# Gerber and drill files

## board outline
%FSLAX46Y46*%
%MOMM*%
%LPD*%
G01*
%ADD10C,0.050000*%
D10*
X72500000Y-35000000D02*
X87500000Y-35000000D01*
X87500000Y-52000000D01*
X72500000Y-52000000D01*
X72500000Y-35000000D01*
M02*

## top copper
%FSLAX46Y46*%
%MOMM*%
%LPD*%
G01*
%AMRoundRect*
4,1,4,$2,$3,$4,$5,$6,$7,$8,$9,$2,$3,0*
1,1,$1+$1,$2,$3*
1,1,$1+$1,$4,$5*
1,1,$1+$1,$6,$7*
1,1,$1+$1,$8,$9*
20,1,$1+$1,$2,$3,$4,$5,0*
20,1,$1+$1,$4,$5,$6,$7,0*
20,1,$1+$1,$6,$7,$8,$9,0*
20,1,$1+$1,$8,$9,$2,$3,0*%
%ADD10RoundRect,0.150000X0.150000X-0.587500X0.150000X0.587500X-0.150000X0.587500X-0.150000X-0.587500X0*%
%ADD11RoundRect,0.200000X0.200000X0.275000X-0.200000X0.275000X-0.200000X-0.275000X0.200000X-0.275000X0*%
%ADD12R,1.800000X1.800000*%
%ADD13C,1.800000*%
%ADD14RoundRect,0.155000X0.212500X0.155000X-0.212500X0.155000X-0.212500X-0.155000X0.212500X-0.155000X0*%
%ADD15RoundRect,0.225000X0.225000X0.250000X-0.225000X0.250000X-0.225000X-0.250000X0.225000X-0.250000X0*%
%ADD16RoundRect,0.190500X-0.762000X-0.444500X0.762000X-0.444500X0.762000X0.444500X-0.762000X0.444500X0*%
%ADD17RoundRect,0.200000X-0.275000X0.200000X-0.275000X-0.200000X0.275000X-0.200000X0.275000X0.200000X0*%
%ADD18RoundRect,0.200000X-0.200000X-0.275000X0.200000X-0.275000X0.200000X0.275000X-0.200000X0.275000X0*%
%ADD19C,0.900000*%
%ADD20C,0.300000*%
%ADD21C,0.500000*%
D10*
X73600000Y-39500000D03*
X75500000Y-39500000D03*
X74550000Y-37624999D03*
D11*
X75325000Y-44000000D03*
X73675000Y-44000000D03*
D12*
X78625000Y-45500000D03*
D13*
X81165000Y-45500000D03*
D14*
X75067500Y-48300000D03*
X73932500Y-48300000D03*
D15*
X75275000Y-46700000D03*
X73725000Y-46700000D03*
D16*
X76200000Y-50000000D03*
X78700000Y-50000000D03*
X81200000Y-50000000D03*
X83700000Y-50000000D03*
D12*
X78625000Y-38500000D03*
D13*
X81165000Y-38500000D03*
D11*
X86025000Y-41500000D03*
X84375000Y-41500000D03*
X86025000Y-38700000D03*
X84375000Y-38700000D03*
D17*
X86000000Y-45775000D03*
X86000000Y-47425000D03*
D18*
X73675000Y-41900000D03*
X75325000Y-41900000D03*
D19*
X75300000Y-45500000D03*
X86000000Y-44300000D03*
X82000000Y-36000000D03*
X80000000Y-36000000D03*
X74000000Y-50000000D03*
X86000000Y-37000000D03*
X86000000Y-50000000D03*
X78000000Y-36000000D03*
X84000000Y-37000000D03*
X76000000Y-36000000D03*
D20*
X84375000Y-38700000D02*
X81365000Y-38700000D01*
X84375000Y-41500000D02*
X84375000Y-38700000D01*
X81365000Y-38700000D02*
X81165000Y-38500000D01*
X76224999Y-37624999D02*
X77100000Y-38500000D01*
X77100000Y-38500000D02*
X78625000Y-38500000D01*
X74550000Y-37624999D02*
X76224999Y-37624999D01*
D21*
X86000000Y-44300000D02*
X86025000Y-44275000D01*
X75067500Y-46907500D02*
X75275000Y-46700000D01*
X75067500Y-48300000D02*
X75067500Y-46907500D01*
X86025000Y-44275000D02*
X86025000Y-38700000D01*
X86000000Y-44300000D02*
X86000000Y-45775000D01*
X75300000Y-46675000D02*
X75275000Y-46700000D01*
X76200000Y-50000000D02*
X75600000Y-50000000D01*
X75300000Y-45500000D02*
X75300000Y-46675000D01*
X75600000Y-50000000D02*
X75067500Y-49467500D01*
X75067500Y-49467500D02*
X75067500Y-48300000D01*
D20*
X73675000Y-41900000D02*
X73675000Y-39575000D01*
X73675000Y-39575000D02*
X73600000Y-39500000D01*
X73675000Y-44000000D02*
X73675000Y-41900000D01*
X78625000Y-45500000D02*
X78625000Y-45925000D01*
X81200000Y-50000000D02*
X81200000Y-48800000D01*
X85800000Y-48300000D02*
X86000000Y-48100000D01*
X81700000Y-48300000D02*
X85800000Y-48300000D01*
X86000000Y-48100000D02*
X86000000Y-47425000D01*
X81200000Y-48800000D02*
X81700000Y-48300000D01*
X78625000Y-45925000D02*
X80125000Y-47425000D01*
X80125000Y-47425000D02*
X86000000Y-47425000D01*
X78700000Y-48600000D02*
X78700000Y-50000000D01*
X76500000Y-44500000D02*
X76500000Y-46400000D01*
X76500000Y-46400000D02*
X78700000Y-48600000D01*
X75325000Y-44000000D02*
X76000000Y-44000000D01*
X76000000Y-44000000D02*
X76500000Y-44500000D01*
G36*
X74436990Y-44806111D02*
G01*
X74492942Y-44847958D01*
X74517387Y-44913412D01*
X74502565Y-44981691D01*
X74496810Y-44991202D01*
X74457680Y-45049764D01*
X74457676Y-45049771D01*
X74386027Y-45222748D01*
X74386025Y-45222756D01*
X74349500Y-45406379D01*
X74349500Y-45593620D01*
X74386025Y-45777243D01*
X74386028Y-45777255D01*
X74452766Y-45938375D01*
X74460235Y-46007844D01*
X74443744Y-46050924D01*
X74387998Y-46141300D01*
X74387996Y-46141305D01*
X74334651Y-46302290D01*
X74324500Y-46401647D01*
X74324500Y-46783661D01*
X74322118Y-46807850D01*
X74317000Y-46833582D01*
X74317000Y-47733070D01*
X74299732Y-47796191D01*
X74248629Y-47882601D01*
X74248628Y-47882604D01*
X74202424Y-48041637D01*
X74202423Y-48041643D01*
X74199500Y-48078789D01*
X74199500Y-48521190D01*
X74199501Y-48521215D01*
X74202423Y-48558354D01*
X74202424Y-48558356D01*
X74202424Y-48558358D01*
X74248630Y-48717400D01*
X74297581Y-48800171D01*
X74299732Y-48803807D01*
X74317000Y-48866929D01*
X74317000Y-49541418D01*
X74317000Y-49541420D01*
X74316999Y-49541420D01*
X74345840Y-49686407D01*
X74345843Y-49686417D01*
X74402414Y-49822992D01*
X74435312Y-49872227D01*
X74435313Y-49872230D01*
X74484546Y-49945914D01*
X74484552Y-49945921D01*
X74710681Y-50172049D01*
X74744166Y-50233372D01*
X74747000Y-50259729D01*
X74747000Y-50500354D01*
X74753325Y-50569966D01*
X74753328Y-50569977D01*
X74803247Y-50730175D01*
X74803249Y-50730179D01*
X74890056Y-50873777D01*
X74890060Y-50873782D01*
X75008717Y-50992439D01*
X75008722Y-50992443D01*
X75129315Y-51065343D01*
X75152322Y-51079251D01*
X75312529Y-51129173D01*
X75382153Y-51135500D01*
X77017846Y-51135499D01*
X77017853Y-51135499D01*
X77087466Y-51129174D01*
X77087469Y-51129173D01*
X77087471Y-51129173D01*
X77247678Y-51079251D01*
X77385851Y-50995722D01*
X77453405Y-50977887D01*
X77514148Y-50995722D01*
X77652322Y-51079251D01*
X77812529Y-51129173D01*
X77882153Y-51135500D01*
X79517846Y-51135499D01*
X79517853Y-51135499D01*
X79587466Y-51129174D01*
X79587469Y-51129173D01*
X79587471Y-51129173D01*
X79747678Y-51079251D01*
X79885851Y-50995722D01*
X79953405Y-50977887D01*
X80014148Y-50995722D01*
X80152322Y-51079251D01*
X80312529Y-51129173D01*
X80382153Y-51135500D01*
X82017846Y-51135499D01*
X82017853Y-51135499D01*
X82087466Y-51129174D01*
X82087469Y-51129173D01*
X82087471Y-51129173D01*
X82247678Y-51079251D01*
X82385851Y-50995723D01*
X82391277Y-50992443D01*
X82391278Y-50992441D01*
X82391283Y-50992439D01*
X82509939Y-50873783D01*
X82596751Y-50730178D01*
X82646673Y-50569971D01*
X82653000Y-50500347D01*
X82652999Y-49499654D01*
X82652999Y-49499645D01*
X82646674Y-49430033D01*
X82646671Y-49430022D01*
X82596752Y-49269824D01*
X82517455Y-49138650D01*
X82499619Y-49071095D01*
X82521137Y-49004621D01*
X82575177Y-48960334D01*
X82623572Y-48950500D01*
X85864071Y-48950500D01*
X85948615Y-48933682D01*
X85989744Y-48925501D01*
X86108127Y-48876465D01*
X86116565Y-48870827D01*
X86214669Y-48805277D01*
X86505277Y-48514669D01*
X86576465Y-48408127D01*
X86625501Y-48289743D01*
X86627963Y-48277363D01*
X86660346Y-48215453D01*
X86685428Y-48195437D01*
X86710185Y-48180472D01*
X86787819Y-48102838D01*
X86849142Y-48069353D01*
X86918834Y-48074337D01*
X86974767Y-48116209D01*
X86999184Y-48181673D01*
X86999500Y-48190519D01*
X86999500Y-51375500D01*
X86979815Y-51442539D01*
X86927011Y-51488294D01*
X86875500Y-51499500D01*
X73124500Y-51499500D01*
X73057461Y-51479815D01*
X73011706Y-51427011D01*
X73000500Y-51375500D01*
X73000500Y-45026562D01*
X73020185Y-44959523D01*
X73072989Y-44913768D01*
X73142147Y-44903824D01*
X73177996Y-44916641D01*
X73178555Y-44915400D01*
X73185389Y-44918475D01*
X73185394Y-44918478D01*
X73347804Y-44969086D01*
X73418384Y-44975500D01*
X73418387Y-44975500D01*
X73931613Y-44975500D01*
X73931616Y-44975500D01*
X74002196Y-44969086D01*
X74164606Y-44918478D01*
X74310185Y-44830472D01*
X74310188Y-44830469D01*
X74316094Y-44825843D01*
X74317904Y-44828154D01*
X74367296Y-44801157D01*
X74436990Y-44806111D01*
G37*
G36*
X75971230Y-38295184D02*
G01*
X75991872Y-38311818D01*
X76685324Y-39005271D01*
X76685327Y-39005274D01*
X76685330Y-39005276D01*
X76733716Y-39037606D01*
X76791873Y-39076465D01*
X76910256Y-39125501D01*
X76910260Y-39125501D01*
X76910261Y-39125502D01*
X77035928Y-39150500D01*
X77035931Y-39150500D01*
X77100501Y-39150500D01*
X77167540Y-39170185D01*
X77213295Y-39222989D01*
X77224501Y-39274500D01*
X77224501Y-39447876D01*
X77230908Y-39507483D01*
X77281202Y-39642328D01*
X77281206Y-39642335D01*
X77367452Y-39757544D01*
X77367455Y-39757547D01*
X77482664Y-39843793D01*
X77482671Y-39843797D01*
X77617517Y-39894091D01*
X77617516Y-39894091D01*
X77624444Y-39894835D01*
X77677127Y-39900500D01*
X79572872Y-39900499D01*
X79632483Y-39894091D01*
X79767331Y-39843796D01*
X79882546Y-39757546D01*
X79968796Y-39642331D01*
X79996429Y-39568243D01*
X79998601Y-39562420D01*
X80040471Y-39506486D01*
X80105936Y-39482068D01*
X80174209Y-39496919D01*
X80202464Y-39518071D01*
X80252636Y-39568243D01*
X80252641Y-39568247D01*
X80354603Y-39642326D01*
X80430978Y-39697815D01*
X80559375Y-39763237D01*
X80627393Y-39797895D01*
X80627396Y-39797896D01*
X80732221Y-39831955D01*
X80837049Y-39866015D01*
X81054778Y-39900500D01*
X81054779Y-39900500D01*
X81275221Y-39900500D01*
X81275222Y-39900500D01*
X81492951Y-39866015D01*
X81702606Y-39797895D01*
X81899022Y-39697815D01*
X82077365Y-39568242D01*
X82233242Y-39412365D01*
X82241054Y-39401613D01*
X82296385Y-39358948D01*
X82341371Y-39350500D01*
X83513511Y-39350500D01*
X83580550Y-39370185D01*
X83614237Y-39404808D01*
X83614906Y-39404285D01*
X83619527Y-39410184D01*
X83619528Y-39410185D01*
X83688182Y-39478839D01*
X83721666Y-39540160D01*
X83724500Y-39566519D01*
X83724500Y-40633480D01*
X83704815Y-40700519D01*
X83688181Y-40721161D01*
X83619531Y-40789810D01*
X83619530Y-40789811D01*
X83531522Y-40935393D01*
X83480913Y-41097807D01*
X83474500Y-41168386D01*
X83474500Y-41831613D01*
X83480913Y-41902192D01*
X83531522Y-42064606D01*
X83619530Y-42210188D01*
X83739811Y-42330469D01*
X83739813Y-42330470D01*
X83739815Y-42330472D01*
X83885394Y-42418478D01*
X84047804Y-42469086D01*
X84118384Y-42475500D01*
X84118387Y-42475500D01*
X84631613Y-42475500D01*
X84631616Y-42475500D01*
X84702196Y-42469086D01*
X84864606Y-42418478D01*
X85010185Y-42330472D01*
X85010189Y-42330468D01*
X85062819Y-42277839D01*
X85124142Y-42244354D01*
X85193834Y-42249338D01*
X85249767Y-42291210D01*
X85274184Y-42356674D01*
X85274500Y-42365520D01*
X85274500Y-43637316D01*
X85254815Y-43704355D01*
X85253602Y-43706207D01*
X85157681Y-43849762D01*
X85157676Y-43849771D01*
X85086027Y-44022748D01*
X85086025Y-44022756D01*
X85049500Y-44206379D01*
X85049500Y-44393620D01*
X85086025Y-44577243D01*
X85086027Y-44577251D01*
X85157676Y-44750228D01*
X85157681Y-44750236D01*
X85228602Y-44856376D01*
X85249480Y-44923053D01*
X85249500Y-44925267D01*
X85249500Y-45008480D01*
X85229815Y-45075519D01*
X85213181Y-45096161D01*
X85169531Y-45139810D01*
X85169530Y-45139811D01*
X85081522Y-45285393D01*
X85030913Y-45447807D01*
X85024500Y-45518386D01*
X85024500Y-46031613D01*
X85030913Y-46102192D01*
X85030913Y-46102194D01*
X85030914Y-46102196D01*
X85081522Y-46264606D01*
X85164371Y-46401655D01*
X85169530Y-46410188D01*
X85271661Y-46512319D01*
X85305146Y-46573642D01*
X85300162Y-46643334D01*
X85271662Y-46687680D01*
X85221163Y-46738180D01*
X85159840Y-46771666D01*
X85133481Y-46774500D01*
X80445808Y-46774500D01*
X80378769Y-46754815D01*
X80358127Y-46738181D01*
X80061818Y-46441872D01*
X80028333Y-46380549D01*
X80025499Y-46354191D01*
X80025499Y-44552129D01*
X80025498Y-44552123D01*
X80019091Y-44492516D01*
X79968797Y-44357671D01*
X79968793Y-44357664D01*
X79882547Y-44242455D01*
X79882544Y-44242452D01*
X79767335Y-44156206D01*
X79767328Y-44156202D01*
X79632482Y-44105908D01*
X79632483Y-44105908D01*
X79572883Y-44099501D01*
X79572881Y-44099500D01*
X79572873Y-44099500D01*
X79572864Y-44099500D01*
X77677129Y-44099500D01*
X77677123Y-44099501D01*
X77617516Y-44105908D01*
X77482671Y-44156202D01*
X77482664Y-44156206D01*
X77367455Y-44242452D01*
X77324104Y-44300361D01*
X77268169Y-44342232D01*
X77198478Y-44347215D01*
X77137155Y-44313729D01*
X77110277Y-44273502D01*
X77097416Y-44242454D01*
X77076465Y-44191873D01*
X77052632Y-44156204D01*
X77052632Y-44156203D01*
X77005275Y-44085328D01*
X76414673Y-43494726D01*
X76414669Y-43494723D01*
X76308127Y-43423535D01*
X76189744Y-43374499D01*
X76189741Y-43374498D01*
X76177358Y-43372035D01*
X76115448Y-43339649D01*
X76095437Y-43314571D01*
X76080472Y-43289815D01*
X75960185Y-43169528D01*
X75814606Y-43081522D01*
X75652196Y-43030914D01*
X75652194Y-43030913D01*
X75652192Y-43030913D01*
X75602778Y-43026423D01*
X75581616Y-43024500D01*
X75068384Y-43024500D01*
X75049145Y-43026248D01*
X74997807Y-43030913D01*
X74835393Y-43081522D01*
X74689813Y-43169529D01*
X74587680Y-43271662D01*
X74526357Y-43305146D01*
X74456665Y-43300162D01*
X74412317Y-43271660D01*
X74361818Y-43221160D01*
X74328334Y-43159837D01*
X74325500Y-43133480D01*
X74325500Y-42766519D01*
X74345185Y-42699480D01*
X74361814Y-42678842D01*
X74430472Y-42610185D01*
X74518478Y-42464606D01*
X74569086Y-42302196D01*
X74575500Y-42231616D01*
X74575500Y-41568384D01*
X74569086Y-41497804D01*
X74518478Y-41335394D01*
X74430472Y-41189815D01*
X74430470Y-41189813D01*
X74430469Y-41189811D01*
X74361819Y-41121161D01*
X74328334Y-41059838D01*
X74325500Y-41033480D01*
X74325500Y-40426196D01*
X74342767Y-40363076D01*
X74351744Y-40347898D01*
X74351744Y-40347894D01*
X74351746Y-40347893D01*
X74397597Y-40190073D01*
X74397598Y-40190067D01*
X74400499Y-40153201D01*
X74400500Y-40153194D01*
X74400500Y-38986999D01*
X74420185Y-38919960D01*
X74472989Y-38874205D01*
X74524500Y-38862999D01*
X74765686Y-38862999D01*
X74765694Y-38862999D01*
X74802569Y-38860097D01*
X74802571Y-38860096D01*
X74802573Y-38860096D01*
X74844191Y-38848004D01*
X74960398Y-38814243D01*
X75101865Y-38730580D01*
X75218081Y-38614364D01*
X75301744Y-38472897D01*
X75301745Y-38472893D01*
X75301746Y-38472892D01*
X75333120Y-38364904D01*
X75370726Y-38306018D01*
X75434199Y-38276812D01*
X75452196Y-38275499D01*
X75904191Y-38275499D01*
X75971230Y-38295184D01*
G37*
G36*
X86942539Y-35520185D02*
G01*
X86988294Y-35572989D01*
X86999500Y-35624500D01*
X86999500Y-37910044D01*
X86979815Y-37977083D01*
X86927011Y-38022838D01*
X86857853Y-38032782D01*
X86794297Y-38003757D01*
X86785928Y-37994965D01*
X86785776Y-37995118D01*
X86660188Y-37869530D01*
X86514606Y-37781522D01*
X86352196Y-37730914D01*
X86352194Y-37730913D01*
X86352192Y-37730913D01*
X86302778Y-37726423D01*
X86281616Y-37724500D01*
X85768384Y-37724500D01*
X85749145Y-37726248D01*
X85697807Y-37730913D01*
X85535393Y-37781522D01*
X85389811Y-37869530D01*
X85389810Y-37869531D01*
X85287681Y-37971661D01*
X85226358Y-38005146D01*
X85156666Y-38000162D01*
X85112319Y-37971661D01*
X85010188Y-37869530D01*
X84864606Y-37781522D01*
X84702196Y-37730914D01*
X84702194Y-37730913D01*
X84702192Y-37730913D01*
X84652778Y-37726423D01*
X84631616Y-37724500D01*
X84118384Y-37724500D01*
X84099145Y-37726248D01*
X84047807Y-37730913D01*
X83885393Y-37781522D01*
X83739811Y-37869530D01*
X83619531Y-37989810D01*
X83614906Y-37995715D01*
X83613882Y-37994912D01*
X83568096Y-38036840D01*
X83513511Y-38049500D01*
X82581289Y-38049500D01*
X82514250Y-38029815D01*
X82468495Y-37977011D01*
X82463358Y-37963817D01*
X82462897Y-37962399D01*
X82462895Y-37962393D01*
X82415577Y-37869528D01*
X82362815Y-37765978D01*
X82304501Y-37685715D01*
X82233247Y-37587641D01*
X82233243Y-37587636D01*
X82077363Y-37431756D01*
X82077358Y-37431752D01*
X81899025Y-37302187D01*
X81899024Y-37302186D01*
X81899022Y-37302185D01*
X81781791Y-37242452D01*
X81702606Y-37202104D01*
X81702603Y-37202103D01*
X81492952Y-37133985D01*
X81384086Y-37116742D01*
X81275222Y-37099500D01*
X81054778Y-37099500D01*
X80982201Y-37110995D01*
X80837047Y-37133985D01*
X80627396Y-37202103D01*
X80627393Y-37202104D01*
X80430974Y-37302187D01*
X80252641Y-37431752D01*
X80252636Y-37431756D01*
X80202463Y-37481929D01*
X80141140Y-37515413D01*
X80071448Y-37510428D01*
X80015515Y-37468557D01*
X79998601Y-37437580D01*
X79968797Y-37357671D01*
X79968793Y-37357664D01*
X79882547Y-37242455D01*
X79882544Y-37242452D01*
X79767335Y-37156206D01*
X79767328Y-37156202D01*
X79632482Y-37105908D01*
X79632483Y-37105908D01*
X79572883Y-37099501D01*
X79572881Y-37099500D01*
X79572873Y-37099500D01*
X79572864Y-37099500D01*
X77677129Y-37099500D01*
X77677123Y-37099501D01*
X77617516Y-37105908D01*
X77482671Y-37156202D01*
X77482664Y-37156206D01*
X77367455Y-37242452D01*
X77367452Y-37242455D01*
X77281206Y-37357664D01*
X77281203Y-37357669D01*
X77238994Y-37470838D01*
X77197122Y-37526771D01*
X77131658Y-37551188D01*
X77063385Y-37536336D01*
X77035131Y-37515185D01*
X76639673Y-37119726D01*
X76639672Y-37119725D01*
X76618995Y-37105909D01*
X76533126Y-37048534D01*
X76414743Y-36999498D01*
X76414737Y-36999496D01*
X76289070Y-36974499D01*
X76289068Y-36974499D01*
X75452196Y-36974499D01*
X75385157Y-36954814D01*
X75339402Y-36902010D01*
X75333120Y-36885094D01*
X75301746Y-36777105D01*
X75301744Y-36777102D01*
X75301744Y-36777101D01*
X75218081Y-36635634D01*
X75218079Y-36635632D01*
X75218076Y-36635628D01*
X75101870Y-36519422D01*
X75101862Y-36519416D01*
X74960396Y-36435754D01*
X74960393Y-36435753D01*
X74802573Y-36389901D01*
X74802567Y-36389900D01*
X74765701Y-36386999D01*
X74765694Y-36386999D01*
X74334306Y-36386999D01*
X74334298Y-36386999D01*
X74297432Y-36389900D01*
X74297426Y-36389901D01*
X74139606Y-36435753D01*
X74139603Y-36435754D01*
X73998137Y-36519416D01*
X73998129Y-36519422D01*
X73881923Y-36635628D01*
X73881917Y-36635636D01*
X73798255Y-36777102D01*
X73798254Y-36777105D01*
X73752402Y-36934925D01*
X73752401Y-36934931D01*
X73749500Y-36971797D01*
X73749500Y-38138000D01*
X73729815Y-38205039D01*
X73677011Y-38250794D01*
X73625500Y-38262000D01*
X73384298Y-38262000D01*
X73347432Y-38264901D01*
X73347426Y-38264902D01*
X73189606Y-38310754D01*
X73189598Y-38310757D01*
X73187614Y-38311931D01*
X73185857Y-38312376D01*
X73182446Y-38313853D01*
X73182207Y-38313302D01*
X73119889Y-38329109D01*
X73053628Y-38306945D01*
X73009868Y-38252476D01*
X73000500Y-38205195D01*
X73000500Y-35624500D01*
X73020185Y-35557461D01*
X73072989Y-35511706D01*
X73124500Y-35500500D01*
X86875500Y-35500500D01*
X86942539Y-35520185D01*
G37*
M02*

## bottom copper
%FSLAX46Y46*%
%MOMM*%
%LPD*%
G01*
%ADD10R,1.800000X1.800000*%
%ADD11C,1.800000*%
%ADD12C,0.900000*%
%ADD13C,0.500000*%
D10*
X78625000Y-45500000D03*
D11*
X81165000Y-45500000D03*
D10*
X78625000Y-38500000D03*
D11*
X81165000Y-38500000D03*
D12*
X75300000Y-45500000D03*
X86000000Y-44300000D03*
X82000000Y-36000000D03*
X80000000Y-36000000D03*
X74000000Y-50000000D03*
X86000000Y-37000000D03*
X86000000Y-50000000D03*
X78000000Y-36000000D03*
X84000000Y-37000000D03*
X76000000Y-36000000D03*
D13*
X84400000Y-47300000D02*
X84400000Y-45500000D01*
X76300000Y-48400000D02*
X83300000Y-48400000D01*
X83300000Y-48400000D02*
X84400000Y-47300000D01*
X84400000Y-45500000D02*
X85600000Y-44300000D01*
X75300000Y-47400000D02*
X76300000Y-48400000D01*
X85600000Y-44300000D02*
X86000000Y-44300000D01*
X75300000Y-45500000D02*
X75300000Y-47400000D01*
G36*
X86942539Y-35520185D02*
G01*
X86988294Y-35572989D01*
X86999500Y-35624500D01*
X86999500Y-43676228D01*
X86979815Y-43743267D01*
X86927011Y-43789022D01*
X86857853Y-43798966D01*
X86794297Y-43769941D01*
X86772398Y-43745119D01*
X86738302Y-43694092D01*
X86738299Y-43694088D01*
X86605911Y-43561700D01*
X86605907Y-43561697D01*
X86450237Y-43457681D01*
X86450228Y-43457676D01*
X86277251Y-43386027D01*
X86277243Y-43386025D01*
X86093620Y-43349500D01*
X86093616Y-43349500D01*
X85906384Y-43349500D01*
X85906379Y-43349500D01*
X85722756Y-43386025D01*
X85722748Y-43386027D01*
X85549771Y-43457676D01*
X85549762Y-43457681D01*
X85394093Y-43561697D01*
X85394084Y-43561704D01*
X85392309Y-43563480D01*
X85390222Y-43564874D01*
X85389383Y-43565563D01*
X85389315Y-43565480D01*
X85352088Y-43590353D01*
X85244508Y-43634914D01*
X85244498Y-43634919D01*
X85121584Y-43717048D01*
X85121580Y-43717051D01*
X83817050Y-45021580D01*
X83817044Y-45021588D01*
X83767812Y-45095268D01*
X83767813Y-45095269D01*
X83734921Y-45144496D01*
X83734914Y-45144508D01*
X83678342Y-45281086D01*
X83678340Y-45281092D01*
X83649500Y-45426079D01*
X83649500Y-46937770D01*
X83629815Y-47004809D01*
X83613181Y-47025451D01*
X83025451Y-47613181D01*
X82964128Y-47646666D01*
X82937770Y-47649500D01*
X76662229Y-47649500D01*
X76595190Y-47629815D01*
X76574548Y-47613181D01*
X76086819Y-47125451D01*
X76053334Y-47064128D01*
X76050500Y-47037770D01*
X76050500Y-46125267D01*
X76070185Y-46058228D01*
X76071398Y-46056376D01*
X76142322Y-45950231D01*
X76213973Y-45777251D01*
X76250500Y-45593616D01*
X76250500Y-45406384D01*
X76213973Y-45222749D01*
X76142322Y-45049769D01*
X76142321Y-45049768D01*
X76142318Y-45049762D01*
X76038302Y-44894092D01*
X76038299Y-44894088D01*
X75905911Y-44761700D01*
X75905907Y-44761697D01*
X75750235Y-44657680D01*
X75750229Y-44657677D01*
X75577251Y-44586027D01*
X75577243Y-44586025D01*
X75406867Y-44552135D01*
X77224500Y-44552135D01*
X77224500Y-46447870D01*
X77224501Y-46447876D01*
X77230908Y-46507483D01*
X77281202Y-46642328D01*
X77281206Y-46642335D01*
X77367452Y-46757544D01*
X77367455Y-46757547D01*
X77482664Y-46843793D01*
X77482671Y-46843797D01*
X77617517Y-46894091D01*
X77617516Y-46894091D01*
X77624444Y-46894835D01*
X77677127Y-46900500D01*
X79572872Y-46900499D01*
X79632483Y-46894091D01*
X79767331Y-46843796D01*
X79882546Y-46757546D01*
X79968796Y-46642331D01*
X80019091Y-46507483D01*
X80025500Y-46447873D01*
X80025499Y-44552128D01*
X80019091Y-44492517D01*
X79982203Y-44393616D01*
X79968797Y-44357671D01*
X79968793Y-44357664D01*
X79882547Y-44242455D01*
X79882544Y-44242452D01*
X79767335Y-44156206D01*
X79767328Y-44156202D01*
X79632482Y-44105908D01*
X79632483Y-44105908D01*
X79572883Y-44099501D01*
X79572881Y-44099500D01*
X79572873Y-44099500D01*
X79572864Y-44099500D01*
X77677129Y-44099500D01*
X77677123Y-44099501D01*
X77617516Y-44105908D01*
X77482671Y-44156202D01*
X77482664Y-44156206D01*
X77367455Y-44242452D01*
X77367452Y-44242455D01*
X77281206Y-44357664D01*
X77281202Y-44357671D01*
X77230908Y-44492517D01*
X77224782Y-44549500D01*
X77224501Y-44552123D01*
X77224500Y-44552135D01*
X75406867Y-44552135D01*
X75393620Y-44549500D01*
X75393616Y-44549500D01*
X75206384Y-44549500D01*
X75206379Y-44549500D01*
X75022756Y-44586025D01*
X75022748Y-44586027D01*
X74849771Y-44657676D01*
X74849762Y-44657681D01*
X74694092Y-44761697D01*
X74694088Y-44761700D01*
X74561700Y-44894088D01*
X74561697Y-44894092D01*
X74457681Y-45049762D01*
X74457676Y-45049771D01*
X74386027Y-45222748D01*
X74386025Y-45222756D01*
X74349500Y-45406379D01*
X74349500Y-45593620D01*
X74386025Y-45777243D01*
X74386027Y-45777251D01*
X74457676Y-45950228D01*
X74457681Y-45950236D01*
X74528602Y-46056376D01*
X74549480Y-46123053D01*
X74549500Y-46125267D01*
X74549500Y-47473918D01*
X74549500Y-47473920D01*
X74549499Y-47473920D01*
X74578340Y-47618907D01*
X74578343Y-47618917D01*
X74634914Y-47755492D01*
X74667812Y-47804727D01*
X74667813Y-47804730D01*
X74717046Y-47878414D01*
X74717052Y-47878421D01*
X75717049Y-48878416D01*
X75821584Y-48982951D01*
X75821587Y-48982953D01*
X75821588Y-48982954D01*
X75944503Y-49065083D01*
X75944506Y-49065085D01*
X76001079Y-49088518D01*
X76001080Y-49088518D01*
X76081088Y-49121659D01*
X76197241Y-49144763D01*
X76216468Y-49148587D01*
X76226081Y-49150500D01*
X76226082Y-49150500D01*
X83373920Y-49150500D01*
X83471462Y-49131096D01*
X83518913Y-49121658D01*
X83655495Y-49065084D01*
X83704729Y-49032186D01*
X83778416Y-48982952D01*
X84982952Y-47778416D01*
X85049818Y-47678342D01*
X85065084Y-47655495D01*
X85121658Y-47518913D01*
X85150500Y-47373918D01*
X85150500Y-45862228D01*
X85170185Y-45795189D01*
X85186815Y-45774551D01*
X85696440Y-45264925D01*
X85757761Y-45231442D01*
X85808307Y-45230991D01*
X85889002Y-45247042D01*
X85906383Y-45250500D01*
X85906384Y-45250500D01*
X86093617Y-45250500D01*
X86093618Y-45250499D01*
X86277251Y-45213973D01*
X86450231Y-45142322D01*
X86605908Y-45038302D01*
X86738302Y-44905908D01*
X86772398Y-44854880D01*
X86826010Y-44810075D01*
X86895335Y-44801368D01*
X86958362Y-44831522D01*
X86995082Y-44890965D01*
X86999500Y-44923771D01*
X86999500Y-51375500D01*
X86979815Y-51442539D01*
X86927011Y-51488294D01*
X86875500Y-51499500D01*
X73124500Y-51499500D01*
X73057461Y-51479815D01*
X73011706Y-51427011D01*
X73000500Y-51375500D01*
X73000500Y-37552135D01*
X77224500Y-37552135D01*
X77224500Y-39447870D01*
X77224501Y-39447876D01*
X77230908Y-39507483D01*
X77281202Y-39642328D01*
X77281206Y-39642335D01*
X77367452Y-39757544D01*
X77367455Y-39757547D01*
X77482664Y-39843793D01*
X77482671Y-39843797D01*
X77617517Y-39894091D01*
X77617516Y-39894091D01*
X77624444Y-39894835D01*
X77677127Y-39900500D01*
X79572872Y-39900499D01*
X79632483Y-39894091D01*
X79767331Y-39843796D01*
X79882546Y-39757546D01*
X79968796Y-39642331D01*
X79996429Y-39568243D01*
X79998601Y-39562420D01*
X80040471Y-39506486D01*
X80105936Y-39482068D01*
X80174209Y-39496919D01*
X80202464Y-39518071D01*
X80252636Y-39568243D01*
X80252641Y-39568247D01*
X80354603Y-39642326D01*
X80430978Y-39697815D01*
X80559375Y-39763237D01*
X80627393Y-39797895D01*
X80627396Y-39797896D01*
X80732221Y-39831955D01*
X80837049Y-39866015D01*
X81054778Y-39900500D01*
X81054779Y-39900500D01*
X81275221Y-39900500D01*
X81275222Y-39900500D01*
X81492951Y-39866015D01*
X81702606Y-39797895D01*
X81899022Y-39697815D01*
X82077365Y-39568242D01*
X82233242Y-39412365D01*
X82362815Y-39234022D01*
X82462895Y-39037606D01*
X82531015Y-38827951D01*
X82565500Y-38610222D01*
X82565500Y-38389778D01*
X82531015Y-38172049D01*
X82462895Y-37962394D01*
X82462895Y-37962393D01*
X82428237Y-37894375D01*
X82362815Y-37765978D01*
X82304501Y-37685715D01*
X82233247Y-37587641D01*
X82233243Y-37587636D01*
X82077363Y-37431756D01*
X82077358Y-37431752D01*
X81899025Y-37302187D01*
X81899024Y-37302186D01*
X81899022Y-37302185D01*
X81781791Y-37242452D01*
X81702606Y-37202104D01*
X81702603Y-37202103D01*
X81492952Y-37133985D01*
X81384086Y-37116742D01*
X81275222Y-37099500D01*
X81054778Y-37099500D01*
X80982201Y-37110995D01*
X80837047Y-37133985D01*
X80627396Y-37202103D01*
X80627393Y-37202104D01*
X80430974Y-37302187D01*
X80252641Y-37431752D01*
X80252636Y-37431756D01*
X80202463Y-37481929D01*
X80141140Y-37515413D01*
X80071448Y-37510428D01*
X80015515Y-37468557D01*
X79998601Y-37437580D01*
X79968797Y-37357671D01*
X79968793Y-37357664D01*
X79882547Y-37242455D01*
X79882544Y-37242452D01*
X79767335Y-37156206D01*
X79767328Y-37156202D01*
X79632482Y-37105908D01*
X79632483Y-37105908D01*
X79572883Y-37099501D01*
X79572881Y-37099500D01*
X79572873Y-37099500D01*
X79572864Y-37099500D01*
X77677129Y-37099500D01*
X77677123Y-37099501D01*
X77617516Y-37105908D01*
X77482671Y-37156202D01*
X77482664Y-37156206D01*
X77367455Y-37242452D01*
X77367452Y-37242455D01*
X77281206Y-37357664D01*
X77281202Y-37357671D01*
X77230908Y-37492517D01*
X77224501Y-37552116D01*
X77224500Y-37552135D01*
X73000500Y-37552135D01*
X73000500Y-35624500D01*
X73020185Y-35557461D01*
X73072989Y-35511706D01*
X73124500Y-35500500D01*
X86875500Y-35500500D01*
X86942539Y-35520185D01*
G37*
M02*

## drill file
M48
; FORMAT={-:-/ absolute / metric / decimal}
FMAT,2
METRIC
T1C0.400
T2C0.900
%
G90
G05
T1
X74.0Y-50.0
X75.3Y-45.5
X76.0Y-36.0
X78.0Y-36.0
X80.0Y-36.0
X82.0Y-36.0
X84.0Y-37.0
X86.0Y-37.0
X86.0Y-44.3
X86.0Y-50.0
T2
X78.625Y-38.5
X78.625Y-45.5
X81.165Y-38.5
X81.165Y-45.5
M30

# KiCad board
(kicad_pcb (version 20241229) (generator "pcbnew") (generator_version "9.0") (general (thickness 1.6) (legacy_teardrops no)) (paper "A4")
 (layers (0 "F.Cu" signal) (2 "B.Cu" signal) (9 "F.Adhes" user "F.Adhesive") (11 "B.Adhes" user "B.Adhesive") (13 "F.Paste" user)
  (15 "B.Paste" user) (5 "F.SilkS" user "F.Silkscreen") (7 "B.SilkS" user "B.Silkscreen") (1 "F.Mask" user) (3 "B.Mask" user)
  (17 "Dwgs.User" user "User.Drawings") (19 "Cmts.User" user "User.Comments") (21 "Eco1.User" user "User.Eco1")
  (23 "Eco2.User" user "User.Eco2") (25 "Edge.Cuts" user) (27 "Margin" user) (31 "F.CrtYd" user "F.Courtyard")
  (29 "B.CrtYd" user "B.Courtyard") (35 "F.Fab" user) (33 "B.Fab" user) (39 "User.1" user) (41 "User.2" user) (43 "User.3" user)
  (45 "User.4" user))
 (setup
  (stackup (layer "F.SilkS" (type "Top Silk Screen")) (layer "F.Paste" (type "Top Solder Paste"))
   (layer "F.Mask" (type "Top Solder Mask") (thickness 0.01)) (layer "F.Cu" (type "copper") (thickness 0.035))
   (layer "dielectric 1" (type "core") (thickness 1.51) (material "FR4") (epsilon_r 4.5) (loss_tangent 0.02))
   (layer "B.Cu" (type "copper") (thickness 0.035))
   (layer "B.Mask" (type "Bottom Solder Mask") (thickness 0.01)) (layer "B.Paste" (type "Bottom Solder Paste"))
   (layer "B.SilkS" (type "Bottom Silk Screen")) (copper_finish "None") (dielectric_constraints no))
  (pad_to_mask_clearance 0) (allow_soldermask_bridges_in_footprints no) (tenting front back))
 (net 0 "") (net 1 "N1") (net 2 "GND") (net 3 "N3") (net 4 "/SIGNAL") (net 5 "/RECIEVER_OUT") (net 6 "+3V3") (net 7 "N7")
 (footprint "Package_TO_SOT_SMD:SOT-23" (layer "F.Cu") (at 74.55 38.5625 90)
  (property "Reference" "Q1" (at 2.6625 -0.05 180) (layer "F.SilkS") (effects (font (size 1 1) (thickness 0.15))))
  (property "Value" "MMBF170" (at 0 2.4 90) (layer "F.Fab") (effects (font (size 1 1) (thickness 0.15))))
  (pad "1" smd roundrect (at -0.9375 -0.95 90) (size 1.475 0.6) (layers "F.Cu" "F.Mask" "F.Paste") (roundrect_rratio 0.25) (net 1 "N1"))
  (pad "2" smd roundrect (at -0.9375 0.95 90) (size 1.475 0.6) (layers "F.Cu" "F.Mask" "F.Paste") (roundrect_rratio 0.25) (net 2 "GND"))
  (pad "3" smd roundrect (at 0.937501 0 90) (size 1.475 0.6) (layers "F.Cu" "F.Mask" "F.Paste") (roundrect_rratio 0.25) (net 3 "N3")))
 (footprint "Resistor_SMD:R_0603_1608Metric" (layer "F.Cu") (at 74.5 44 180)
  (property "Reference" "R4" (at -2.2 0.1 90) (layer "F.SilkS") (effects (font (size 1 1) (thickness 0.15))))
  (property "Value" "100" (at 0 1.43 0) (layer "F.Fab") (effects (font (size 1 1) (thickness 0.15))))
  (pad "1" smd roundrect (at -0.825 0 180) (size 0.8 0.95) (layers "F.Cu" "F.Mask" "F.Paste") (roundrect_rratio 0.25) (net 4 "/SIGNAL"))
  (pad "2" smd roundrect (at 0.825 0 180) (size 0.8 0.95) (layers "F.Cu" "F.Mask" "F.Paste") (roundrect_rratio 0.25) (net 1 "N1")))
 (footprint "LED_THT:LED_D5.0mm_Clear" (layer "F.Cu") (at 78.625 45.5)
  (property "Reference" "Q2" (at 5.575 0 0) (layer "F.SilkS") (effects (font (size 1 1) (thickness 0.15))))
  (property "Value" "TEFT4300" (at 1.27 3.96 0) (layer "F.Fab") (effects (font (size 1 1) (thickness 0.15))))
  (pad "1" thru_hole rect (at 0 0) (size 1.8 1.8) (drill 0.9) (layers "*.Cu" "*.Mask") (remove_unused_layers no) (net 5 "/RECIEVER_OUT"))
  (pad "2" thru_hole circle (at 2.54 0) (size 1.8 1.8) (drill 0.9) (layers "*.Cu" "*.Mask") (remove_unused_layers no) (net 2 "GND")))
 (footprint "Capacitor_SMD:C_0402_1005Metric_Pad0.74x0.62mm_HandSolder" (layer "F.Cu") (at 74.5 48.3 180)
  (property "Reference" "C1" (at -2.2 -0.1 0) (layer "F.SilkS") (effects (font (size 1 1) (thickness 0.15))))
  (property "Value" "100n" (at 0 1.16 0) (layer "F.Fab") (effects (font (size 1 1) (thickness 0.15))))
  (pad "1" smd roundrect (at -0.5675 0 180) (size 0.735 0.62) (layers "F.Cu" "F.Mask" "F.Paste") (roundrect_rratio 0.25) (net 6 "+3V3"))
  (pad "2" smd roundrect (at 0.5675 0 180) (size 0.735 0.62) (layers "F.Cu" "F.Mask" "F.Paste") (roundrect_rratio 0.25) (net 2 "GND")))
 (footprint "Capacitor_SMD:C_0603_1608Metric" (layer "F.Cu") (at 74.5 46.7 180)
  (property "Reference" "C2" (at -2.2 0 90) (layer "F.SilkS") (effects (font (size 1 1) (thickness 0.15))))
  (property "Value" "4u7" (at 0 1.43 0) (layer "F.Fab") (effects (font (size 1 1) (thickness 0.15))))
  (pad "1" smd roundrect (at -0.775 0 180) (size 0.9 0.95) (layers "F.Cu" "F.Mask" "F.Paste") (roundrect_rratio 0.25) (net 6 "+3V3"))
  (pad "2" smd roundrect (at 0.775 0 180) (size 0.9 0.95) (layers "F.Cu" "F.Mask" "F.Paste") (roundrect_rratio 0.25) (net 2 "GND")))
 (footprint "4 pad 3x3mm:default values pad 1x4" (layer "F.Cu") (at 80.2 45)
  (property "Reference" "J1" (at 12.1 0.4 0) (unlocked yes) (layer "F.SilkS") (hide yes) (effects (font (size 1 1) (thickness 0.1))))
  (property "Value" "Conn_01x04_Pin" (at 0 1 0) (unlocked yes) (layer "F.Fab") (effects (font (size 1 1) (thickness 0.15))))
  (pad "1" smd roundrect (at -4 5) (size 1.905 1.27) (layers "F.Cu" "F.Mask" "F.Paste") (roundrect_rratio 0.15) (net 6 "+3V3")
   (thermal_bridge_angle 45))
  (pad "2" smd roundrect (at -1.5 5) (size 1.905 1.27) (layers "F.Cu" "F.Mask" "F.Paste") (roundrect_rratio 0.15) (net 4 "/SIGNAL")
   (thermal_bridge_angle 45))
  (pad "3" smd roundrect (at 1 5) (size 1.905 1.27) (layers "F.Cu" "F.Mask" "F.Paste") (roundrect_rratio 0.15) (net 5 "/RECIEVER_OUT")
   (thermal_bridge_angle 45))
  (pad "4" smd roundrect (at 3.5 5) (size 1.905 1.27) (layers "F.Cu" "F.Mask" "F.Paste") (roundrect_rratio 0.15) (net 2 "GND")
   (thermal_bridge_angle 45)))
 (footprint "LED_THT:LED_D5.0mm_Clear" (layer "F.Cu") (at 78.625 38.5)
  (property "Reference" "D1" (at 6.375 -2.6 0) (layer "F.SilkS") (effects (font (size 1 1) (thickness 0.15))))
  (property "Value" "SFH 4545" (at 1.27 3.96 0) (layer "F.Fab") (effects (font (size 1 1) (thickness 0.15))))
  (pad "1" thru_hole rect (at 0 0) (size 1.8 1.8) (drill 0.9) (layers "*.Cu" "*.Mask") (remove_unused_layers no) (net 3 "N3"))
  (pad "2" thru_hole circle (at 2.54 0) (size 1.8 1.8) (drill 0.9) (layers "*.Cu" "*.Mask") (remove_unused_layers no) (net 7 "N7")))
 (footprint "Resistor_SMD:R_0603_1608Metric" (layer "F.Cu") (at 85.2 41.5 180)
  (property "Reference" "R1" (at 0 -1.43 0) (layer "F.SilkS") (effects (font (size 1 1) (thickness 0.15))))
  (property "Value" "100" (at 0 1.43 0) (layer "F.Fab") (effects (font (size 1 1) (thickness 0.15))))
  (pad "1" smd roundrect (at -0.825 0 180) (size 0.8 0.95) (layers "F.Cu" "F.Mask" "F.Paste") (roundrect_rratio 0.25) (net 6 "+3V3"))
  (pad "2" smd roundrect (at 0.825 0 180) (size 0.8 0.95) (layers "F.Cu" "F.Mask" "F.Paste") (roundrect_rratio 0.25) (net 7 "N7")))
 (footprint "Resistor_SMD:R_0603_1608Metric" (layer "F.Cu") (at 85.2 38.7 180)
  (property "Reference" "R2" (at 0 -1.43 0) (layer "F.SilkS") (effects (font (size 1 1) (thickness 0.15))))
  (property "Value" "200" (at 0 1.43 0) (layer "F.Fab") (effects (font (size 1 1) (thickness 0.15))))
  (pad "1" smd roundrect (at -0.825 0 180) (size 0.8 0.95) (layers "F.Cu" "F.Mask" "F.Paste") (roundrect_rratio 0.25) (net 6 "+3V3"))
  (pad "2" smd roundrect (at 0.825 0 180) (size 0.8 0.95) (layers "F.Cu" "F.Mask" "F.Paste") (roundrect_rratio 0.25) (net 7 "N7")))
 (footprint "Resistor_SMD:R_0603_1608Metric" (layer "F.Cu") (at 86 46.6 -90)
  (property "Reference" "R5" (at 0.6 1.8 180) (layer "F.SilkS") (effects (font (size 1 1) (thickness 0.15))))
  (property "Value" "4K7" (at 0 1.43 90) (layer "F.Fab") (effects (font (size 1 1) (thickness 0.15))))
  (pad "1" smd roundrect (at -0.825 0 270) (size 0.8 0.95) (layers "F.Cu" "F.Mask" "F.Paste") (roundrect_rratio 0.25) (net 6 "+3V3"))
  (pad "2" smd roundrect (at 0.825 0 270) (size 0.8 0.95) (layers "F.Cu" "F.Mask" "F.Paste") (roundrect_rratio 0.25) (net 5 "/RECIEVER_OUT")))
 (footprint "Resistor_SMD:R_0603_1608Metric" (layer "F.Cu") (at 74.5 41.9)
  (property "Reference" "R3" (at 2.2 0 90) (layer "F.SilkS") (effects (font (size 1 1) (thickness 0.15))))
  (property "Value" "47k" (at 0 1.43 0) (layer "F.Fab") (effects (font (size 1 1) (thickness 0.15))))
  (pad "1" smd roundrect (at -0.825 0) (size 0.8 0.95) (layers "F.Cu" "F.Mask" "F.Paste") (roundrect_rratio 0.25) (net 1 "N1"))
  (pad "2" smd roundrect (at 0.825 0) (size 0.8 0.95) (layers "F.Cu" "F.Mask" "F.Paste") (roundrect_rratio 0.25) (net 2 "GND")))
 (gr_rect (start 72.5 35) (end 87.5 52) (stroke (width 0.05) (type default)) (fill no) (layer "Edge.Cuts"))
 (segment (start 84.375 38.7) (end 81.365 38.7) (width 0.3) (layer "F.Cu") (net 7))
 (segment (start 84.375 41.5) (end 84.375 38.7) (width 0.3) (layer "F.Cu") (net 7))
 (segment (start 81.365 38.7) (end 81.165 38.5) (width 0.3) (layer "F.Cu") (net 7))
 (segment (start 76.224999 37.624999) (end 77.1 38.5) (width 0.3) (layer "F.Cu") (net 3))
 (segment (start 77.1 38.5) (end 78.625 38.5) (width 0.3) (layer "F.Cu") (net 3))
 (segment (start 74.55 37.624999) (end 76.224999 37.624999) (width 0.3) (layer "F.Cu") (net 3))
 (segment (start 86 44.3) (end 86.025 44.275) (width 0.5) (layer "F.Cu") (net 6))
 (segment (start 75.0675 46.9075) (end 75.275 46.7) (width 0.5) (layer "F.Cu") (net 6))
 (segment (start 75.0675 48.3) (end 75.0675 46.9075) (width 0.5) (layer "F.Cu") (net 6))
 (segment (start 86.025 44.275) (end 86.025 38.7) (width 0.5) (layer "F.Cu") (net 6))
 (segment (start 86 44.3) (end 86 45.775) (width 0.5) (layer "F.Cu") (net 6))
 (segment (start 75.3 46.675) (end 75.275 46.7) (width 0.5) (layer "F.Cu") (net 6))
 (segment (start 76.2 50) (end 75.6 50) (width 0.5) (layer "F.Cu") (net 6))
 (segment (start 75.3 45.5) (end 75.3 46.675) (width 0.5) (layer "F.Cu") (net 6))
 (segment (start 75.6 50) (end 75.0675 49.4675) (width 0.5) (layer "F.Cu") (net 6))
 (segment (start 75.0675 49.4675) (end 75.0675 48.3) (width 0.5) (layer "F.Cu") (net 6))
 (via (at 75.3 45.5) (size 0.9) (drill 0.4) (layers "F.Cu" "B.Cu") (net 6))
 (via (at 86 44.3) (size 0.9) (drill 0.4) (layers "F.Cu" "B.Cu") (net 6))
 (segment (start 84.4 47.3) (end 84.4 45.5) (width 0.5) (layer "B.Cu") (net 6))
 (segment (start 76.3 48.4) (end 83.3 48.4) (width 0.5) (layer "B.Cu") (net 6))
 (segment (start 83.3 48.4) (end 84.4 47.3) (width 0.5) (layer "B.Cu") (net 6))
 (segment (start 84.4 45.5) (end 85.6 44.3) (width 0.5) (layer "B.Cu") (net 6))
 (segment (start 75.3 47.4) (end 76.3 48.4) (width 0.5) (layer "B.Cu") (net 6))
 (segment (start 85.6 44.3) (end 86 44.3) (width 0.5) (layer "B.Cu") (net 6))
 (segment (start 75.3 45.5) (end 75.3 47.4) (width 0.5) (layer "B.Cu") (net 6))
 (segment (start 73.675 41.9) (end 73.675 39.575) (width 0.3) (layer "F.Cu") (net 1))
 (segment (start 73.675 39.575) (end 73.6 39.5) (width 0.3) (layer "F.Cu") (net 1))
 (segment (start 73.675 44) (end 73.675 41.9) (width 0.3) (layer "F.Cu") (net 1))
 (via (at 82 36) (size 0.9) (drill 0.4) (layers "F.Cu" "B.Cu") (free yes) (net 2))
 (via (at 80 36) (size 0.9) (drill 0.4) (layers "F.Cu" "B.Cu") (free yes) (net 2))
 (via (at 74 50) (size 0.9) (drill 0.4) (layers "F.Cu" "B.Cu") (free yes) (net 2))
 (via (at 86 37) (size 0.9) (drill 0.4) (layers "F.Cu" "B.Cu") (free yes) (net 2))
 (via (at 86 50) (size 0.9) (drill 0.4) (layers "F.Cu" "B.Cu") (free yes) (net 2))
 (via (at 78 36) (size 0.9) (drill 0.4) (layers "F.Cu" "B.Cu") (free yes) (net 2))
 (via (at 84 37) (size 0.9) (drill 0.4) (layers "F.Cu" "B.Cu") (free yes) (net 2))
 (via (at 76 36) (size 0.9) (drill 0.4) (layers "F.Cu" "B.Cu") (free yes) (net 2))
 (segment (start 78.625 45.5) (end 78.625 45.925) (width 0.3) (layer "F.Cu") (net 5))
 (segment (start 81.2 50) (end 81.2 48.8) (width 0.3) (layer "F.Cu") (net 5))
 (segment (start 85.8 48.3) (end 86 48.1) (width 0.3) (layer "F.Cu") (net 5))
 (segment (start 81.7 48.3) (end 85.8 48.3) (width 0.3) (layer "F.Cu") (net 5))
 (segment (start 86 48.1) (end 86 47.425) (width 0.3) (layer "F.Cu") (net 5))
 (segment (start 81.2 48.8) (end 81.7 48.3) (width 0.3) (layer "F.Cu") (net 5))
 (segment (start 78.625 45.925) (end 80.125 47.425) (width 0.3) (layer "F.Cu") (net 5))
 (segment (start 80.125 47.425) (end 86 47.425) (width 0.3) (layer "F.Cu") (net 5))
 (segment (start 78.7 48.6) (end 78.7 50) (width 0.3) (layer "F.Cu") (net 4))
 (segment (start 76.5 44.5) (end 76.5 46.4) (width 0.3) (layer "F.Cu") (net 4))
 (segment (start 76.5 46.4) (end 78.7 48.6) (width 0.3) (layer "F.Cu") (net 4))
 (segment (start 75.325 44) (end 76 44) (width 0.3) (layer "F.Cu") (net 4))
 (segment (start 76 44) (end 76.5 44.5) (width 0.3) (layer "F.Cu") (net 4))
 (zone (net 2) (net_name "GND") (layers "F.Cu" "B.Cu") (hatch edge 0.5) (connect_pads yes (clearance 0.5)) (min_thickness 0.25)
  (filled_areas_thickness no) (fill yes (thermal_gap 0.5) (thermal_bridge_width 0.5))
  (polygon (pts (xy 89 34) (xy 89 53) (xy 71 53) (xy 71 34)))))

